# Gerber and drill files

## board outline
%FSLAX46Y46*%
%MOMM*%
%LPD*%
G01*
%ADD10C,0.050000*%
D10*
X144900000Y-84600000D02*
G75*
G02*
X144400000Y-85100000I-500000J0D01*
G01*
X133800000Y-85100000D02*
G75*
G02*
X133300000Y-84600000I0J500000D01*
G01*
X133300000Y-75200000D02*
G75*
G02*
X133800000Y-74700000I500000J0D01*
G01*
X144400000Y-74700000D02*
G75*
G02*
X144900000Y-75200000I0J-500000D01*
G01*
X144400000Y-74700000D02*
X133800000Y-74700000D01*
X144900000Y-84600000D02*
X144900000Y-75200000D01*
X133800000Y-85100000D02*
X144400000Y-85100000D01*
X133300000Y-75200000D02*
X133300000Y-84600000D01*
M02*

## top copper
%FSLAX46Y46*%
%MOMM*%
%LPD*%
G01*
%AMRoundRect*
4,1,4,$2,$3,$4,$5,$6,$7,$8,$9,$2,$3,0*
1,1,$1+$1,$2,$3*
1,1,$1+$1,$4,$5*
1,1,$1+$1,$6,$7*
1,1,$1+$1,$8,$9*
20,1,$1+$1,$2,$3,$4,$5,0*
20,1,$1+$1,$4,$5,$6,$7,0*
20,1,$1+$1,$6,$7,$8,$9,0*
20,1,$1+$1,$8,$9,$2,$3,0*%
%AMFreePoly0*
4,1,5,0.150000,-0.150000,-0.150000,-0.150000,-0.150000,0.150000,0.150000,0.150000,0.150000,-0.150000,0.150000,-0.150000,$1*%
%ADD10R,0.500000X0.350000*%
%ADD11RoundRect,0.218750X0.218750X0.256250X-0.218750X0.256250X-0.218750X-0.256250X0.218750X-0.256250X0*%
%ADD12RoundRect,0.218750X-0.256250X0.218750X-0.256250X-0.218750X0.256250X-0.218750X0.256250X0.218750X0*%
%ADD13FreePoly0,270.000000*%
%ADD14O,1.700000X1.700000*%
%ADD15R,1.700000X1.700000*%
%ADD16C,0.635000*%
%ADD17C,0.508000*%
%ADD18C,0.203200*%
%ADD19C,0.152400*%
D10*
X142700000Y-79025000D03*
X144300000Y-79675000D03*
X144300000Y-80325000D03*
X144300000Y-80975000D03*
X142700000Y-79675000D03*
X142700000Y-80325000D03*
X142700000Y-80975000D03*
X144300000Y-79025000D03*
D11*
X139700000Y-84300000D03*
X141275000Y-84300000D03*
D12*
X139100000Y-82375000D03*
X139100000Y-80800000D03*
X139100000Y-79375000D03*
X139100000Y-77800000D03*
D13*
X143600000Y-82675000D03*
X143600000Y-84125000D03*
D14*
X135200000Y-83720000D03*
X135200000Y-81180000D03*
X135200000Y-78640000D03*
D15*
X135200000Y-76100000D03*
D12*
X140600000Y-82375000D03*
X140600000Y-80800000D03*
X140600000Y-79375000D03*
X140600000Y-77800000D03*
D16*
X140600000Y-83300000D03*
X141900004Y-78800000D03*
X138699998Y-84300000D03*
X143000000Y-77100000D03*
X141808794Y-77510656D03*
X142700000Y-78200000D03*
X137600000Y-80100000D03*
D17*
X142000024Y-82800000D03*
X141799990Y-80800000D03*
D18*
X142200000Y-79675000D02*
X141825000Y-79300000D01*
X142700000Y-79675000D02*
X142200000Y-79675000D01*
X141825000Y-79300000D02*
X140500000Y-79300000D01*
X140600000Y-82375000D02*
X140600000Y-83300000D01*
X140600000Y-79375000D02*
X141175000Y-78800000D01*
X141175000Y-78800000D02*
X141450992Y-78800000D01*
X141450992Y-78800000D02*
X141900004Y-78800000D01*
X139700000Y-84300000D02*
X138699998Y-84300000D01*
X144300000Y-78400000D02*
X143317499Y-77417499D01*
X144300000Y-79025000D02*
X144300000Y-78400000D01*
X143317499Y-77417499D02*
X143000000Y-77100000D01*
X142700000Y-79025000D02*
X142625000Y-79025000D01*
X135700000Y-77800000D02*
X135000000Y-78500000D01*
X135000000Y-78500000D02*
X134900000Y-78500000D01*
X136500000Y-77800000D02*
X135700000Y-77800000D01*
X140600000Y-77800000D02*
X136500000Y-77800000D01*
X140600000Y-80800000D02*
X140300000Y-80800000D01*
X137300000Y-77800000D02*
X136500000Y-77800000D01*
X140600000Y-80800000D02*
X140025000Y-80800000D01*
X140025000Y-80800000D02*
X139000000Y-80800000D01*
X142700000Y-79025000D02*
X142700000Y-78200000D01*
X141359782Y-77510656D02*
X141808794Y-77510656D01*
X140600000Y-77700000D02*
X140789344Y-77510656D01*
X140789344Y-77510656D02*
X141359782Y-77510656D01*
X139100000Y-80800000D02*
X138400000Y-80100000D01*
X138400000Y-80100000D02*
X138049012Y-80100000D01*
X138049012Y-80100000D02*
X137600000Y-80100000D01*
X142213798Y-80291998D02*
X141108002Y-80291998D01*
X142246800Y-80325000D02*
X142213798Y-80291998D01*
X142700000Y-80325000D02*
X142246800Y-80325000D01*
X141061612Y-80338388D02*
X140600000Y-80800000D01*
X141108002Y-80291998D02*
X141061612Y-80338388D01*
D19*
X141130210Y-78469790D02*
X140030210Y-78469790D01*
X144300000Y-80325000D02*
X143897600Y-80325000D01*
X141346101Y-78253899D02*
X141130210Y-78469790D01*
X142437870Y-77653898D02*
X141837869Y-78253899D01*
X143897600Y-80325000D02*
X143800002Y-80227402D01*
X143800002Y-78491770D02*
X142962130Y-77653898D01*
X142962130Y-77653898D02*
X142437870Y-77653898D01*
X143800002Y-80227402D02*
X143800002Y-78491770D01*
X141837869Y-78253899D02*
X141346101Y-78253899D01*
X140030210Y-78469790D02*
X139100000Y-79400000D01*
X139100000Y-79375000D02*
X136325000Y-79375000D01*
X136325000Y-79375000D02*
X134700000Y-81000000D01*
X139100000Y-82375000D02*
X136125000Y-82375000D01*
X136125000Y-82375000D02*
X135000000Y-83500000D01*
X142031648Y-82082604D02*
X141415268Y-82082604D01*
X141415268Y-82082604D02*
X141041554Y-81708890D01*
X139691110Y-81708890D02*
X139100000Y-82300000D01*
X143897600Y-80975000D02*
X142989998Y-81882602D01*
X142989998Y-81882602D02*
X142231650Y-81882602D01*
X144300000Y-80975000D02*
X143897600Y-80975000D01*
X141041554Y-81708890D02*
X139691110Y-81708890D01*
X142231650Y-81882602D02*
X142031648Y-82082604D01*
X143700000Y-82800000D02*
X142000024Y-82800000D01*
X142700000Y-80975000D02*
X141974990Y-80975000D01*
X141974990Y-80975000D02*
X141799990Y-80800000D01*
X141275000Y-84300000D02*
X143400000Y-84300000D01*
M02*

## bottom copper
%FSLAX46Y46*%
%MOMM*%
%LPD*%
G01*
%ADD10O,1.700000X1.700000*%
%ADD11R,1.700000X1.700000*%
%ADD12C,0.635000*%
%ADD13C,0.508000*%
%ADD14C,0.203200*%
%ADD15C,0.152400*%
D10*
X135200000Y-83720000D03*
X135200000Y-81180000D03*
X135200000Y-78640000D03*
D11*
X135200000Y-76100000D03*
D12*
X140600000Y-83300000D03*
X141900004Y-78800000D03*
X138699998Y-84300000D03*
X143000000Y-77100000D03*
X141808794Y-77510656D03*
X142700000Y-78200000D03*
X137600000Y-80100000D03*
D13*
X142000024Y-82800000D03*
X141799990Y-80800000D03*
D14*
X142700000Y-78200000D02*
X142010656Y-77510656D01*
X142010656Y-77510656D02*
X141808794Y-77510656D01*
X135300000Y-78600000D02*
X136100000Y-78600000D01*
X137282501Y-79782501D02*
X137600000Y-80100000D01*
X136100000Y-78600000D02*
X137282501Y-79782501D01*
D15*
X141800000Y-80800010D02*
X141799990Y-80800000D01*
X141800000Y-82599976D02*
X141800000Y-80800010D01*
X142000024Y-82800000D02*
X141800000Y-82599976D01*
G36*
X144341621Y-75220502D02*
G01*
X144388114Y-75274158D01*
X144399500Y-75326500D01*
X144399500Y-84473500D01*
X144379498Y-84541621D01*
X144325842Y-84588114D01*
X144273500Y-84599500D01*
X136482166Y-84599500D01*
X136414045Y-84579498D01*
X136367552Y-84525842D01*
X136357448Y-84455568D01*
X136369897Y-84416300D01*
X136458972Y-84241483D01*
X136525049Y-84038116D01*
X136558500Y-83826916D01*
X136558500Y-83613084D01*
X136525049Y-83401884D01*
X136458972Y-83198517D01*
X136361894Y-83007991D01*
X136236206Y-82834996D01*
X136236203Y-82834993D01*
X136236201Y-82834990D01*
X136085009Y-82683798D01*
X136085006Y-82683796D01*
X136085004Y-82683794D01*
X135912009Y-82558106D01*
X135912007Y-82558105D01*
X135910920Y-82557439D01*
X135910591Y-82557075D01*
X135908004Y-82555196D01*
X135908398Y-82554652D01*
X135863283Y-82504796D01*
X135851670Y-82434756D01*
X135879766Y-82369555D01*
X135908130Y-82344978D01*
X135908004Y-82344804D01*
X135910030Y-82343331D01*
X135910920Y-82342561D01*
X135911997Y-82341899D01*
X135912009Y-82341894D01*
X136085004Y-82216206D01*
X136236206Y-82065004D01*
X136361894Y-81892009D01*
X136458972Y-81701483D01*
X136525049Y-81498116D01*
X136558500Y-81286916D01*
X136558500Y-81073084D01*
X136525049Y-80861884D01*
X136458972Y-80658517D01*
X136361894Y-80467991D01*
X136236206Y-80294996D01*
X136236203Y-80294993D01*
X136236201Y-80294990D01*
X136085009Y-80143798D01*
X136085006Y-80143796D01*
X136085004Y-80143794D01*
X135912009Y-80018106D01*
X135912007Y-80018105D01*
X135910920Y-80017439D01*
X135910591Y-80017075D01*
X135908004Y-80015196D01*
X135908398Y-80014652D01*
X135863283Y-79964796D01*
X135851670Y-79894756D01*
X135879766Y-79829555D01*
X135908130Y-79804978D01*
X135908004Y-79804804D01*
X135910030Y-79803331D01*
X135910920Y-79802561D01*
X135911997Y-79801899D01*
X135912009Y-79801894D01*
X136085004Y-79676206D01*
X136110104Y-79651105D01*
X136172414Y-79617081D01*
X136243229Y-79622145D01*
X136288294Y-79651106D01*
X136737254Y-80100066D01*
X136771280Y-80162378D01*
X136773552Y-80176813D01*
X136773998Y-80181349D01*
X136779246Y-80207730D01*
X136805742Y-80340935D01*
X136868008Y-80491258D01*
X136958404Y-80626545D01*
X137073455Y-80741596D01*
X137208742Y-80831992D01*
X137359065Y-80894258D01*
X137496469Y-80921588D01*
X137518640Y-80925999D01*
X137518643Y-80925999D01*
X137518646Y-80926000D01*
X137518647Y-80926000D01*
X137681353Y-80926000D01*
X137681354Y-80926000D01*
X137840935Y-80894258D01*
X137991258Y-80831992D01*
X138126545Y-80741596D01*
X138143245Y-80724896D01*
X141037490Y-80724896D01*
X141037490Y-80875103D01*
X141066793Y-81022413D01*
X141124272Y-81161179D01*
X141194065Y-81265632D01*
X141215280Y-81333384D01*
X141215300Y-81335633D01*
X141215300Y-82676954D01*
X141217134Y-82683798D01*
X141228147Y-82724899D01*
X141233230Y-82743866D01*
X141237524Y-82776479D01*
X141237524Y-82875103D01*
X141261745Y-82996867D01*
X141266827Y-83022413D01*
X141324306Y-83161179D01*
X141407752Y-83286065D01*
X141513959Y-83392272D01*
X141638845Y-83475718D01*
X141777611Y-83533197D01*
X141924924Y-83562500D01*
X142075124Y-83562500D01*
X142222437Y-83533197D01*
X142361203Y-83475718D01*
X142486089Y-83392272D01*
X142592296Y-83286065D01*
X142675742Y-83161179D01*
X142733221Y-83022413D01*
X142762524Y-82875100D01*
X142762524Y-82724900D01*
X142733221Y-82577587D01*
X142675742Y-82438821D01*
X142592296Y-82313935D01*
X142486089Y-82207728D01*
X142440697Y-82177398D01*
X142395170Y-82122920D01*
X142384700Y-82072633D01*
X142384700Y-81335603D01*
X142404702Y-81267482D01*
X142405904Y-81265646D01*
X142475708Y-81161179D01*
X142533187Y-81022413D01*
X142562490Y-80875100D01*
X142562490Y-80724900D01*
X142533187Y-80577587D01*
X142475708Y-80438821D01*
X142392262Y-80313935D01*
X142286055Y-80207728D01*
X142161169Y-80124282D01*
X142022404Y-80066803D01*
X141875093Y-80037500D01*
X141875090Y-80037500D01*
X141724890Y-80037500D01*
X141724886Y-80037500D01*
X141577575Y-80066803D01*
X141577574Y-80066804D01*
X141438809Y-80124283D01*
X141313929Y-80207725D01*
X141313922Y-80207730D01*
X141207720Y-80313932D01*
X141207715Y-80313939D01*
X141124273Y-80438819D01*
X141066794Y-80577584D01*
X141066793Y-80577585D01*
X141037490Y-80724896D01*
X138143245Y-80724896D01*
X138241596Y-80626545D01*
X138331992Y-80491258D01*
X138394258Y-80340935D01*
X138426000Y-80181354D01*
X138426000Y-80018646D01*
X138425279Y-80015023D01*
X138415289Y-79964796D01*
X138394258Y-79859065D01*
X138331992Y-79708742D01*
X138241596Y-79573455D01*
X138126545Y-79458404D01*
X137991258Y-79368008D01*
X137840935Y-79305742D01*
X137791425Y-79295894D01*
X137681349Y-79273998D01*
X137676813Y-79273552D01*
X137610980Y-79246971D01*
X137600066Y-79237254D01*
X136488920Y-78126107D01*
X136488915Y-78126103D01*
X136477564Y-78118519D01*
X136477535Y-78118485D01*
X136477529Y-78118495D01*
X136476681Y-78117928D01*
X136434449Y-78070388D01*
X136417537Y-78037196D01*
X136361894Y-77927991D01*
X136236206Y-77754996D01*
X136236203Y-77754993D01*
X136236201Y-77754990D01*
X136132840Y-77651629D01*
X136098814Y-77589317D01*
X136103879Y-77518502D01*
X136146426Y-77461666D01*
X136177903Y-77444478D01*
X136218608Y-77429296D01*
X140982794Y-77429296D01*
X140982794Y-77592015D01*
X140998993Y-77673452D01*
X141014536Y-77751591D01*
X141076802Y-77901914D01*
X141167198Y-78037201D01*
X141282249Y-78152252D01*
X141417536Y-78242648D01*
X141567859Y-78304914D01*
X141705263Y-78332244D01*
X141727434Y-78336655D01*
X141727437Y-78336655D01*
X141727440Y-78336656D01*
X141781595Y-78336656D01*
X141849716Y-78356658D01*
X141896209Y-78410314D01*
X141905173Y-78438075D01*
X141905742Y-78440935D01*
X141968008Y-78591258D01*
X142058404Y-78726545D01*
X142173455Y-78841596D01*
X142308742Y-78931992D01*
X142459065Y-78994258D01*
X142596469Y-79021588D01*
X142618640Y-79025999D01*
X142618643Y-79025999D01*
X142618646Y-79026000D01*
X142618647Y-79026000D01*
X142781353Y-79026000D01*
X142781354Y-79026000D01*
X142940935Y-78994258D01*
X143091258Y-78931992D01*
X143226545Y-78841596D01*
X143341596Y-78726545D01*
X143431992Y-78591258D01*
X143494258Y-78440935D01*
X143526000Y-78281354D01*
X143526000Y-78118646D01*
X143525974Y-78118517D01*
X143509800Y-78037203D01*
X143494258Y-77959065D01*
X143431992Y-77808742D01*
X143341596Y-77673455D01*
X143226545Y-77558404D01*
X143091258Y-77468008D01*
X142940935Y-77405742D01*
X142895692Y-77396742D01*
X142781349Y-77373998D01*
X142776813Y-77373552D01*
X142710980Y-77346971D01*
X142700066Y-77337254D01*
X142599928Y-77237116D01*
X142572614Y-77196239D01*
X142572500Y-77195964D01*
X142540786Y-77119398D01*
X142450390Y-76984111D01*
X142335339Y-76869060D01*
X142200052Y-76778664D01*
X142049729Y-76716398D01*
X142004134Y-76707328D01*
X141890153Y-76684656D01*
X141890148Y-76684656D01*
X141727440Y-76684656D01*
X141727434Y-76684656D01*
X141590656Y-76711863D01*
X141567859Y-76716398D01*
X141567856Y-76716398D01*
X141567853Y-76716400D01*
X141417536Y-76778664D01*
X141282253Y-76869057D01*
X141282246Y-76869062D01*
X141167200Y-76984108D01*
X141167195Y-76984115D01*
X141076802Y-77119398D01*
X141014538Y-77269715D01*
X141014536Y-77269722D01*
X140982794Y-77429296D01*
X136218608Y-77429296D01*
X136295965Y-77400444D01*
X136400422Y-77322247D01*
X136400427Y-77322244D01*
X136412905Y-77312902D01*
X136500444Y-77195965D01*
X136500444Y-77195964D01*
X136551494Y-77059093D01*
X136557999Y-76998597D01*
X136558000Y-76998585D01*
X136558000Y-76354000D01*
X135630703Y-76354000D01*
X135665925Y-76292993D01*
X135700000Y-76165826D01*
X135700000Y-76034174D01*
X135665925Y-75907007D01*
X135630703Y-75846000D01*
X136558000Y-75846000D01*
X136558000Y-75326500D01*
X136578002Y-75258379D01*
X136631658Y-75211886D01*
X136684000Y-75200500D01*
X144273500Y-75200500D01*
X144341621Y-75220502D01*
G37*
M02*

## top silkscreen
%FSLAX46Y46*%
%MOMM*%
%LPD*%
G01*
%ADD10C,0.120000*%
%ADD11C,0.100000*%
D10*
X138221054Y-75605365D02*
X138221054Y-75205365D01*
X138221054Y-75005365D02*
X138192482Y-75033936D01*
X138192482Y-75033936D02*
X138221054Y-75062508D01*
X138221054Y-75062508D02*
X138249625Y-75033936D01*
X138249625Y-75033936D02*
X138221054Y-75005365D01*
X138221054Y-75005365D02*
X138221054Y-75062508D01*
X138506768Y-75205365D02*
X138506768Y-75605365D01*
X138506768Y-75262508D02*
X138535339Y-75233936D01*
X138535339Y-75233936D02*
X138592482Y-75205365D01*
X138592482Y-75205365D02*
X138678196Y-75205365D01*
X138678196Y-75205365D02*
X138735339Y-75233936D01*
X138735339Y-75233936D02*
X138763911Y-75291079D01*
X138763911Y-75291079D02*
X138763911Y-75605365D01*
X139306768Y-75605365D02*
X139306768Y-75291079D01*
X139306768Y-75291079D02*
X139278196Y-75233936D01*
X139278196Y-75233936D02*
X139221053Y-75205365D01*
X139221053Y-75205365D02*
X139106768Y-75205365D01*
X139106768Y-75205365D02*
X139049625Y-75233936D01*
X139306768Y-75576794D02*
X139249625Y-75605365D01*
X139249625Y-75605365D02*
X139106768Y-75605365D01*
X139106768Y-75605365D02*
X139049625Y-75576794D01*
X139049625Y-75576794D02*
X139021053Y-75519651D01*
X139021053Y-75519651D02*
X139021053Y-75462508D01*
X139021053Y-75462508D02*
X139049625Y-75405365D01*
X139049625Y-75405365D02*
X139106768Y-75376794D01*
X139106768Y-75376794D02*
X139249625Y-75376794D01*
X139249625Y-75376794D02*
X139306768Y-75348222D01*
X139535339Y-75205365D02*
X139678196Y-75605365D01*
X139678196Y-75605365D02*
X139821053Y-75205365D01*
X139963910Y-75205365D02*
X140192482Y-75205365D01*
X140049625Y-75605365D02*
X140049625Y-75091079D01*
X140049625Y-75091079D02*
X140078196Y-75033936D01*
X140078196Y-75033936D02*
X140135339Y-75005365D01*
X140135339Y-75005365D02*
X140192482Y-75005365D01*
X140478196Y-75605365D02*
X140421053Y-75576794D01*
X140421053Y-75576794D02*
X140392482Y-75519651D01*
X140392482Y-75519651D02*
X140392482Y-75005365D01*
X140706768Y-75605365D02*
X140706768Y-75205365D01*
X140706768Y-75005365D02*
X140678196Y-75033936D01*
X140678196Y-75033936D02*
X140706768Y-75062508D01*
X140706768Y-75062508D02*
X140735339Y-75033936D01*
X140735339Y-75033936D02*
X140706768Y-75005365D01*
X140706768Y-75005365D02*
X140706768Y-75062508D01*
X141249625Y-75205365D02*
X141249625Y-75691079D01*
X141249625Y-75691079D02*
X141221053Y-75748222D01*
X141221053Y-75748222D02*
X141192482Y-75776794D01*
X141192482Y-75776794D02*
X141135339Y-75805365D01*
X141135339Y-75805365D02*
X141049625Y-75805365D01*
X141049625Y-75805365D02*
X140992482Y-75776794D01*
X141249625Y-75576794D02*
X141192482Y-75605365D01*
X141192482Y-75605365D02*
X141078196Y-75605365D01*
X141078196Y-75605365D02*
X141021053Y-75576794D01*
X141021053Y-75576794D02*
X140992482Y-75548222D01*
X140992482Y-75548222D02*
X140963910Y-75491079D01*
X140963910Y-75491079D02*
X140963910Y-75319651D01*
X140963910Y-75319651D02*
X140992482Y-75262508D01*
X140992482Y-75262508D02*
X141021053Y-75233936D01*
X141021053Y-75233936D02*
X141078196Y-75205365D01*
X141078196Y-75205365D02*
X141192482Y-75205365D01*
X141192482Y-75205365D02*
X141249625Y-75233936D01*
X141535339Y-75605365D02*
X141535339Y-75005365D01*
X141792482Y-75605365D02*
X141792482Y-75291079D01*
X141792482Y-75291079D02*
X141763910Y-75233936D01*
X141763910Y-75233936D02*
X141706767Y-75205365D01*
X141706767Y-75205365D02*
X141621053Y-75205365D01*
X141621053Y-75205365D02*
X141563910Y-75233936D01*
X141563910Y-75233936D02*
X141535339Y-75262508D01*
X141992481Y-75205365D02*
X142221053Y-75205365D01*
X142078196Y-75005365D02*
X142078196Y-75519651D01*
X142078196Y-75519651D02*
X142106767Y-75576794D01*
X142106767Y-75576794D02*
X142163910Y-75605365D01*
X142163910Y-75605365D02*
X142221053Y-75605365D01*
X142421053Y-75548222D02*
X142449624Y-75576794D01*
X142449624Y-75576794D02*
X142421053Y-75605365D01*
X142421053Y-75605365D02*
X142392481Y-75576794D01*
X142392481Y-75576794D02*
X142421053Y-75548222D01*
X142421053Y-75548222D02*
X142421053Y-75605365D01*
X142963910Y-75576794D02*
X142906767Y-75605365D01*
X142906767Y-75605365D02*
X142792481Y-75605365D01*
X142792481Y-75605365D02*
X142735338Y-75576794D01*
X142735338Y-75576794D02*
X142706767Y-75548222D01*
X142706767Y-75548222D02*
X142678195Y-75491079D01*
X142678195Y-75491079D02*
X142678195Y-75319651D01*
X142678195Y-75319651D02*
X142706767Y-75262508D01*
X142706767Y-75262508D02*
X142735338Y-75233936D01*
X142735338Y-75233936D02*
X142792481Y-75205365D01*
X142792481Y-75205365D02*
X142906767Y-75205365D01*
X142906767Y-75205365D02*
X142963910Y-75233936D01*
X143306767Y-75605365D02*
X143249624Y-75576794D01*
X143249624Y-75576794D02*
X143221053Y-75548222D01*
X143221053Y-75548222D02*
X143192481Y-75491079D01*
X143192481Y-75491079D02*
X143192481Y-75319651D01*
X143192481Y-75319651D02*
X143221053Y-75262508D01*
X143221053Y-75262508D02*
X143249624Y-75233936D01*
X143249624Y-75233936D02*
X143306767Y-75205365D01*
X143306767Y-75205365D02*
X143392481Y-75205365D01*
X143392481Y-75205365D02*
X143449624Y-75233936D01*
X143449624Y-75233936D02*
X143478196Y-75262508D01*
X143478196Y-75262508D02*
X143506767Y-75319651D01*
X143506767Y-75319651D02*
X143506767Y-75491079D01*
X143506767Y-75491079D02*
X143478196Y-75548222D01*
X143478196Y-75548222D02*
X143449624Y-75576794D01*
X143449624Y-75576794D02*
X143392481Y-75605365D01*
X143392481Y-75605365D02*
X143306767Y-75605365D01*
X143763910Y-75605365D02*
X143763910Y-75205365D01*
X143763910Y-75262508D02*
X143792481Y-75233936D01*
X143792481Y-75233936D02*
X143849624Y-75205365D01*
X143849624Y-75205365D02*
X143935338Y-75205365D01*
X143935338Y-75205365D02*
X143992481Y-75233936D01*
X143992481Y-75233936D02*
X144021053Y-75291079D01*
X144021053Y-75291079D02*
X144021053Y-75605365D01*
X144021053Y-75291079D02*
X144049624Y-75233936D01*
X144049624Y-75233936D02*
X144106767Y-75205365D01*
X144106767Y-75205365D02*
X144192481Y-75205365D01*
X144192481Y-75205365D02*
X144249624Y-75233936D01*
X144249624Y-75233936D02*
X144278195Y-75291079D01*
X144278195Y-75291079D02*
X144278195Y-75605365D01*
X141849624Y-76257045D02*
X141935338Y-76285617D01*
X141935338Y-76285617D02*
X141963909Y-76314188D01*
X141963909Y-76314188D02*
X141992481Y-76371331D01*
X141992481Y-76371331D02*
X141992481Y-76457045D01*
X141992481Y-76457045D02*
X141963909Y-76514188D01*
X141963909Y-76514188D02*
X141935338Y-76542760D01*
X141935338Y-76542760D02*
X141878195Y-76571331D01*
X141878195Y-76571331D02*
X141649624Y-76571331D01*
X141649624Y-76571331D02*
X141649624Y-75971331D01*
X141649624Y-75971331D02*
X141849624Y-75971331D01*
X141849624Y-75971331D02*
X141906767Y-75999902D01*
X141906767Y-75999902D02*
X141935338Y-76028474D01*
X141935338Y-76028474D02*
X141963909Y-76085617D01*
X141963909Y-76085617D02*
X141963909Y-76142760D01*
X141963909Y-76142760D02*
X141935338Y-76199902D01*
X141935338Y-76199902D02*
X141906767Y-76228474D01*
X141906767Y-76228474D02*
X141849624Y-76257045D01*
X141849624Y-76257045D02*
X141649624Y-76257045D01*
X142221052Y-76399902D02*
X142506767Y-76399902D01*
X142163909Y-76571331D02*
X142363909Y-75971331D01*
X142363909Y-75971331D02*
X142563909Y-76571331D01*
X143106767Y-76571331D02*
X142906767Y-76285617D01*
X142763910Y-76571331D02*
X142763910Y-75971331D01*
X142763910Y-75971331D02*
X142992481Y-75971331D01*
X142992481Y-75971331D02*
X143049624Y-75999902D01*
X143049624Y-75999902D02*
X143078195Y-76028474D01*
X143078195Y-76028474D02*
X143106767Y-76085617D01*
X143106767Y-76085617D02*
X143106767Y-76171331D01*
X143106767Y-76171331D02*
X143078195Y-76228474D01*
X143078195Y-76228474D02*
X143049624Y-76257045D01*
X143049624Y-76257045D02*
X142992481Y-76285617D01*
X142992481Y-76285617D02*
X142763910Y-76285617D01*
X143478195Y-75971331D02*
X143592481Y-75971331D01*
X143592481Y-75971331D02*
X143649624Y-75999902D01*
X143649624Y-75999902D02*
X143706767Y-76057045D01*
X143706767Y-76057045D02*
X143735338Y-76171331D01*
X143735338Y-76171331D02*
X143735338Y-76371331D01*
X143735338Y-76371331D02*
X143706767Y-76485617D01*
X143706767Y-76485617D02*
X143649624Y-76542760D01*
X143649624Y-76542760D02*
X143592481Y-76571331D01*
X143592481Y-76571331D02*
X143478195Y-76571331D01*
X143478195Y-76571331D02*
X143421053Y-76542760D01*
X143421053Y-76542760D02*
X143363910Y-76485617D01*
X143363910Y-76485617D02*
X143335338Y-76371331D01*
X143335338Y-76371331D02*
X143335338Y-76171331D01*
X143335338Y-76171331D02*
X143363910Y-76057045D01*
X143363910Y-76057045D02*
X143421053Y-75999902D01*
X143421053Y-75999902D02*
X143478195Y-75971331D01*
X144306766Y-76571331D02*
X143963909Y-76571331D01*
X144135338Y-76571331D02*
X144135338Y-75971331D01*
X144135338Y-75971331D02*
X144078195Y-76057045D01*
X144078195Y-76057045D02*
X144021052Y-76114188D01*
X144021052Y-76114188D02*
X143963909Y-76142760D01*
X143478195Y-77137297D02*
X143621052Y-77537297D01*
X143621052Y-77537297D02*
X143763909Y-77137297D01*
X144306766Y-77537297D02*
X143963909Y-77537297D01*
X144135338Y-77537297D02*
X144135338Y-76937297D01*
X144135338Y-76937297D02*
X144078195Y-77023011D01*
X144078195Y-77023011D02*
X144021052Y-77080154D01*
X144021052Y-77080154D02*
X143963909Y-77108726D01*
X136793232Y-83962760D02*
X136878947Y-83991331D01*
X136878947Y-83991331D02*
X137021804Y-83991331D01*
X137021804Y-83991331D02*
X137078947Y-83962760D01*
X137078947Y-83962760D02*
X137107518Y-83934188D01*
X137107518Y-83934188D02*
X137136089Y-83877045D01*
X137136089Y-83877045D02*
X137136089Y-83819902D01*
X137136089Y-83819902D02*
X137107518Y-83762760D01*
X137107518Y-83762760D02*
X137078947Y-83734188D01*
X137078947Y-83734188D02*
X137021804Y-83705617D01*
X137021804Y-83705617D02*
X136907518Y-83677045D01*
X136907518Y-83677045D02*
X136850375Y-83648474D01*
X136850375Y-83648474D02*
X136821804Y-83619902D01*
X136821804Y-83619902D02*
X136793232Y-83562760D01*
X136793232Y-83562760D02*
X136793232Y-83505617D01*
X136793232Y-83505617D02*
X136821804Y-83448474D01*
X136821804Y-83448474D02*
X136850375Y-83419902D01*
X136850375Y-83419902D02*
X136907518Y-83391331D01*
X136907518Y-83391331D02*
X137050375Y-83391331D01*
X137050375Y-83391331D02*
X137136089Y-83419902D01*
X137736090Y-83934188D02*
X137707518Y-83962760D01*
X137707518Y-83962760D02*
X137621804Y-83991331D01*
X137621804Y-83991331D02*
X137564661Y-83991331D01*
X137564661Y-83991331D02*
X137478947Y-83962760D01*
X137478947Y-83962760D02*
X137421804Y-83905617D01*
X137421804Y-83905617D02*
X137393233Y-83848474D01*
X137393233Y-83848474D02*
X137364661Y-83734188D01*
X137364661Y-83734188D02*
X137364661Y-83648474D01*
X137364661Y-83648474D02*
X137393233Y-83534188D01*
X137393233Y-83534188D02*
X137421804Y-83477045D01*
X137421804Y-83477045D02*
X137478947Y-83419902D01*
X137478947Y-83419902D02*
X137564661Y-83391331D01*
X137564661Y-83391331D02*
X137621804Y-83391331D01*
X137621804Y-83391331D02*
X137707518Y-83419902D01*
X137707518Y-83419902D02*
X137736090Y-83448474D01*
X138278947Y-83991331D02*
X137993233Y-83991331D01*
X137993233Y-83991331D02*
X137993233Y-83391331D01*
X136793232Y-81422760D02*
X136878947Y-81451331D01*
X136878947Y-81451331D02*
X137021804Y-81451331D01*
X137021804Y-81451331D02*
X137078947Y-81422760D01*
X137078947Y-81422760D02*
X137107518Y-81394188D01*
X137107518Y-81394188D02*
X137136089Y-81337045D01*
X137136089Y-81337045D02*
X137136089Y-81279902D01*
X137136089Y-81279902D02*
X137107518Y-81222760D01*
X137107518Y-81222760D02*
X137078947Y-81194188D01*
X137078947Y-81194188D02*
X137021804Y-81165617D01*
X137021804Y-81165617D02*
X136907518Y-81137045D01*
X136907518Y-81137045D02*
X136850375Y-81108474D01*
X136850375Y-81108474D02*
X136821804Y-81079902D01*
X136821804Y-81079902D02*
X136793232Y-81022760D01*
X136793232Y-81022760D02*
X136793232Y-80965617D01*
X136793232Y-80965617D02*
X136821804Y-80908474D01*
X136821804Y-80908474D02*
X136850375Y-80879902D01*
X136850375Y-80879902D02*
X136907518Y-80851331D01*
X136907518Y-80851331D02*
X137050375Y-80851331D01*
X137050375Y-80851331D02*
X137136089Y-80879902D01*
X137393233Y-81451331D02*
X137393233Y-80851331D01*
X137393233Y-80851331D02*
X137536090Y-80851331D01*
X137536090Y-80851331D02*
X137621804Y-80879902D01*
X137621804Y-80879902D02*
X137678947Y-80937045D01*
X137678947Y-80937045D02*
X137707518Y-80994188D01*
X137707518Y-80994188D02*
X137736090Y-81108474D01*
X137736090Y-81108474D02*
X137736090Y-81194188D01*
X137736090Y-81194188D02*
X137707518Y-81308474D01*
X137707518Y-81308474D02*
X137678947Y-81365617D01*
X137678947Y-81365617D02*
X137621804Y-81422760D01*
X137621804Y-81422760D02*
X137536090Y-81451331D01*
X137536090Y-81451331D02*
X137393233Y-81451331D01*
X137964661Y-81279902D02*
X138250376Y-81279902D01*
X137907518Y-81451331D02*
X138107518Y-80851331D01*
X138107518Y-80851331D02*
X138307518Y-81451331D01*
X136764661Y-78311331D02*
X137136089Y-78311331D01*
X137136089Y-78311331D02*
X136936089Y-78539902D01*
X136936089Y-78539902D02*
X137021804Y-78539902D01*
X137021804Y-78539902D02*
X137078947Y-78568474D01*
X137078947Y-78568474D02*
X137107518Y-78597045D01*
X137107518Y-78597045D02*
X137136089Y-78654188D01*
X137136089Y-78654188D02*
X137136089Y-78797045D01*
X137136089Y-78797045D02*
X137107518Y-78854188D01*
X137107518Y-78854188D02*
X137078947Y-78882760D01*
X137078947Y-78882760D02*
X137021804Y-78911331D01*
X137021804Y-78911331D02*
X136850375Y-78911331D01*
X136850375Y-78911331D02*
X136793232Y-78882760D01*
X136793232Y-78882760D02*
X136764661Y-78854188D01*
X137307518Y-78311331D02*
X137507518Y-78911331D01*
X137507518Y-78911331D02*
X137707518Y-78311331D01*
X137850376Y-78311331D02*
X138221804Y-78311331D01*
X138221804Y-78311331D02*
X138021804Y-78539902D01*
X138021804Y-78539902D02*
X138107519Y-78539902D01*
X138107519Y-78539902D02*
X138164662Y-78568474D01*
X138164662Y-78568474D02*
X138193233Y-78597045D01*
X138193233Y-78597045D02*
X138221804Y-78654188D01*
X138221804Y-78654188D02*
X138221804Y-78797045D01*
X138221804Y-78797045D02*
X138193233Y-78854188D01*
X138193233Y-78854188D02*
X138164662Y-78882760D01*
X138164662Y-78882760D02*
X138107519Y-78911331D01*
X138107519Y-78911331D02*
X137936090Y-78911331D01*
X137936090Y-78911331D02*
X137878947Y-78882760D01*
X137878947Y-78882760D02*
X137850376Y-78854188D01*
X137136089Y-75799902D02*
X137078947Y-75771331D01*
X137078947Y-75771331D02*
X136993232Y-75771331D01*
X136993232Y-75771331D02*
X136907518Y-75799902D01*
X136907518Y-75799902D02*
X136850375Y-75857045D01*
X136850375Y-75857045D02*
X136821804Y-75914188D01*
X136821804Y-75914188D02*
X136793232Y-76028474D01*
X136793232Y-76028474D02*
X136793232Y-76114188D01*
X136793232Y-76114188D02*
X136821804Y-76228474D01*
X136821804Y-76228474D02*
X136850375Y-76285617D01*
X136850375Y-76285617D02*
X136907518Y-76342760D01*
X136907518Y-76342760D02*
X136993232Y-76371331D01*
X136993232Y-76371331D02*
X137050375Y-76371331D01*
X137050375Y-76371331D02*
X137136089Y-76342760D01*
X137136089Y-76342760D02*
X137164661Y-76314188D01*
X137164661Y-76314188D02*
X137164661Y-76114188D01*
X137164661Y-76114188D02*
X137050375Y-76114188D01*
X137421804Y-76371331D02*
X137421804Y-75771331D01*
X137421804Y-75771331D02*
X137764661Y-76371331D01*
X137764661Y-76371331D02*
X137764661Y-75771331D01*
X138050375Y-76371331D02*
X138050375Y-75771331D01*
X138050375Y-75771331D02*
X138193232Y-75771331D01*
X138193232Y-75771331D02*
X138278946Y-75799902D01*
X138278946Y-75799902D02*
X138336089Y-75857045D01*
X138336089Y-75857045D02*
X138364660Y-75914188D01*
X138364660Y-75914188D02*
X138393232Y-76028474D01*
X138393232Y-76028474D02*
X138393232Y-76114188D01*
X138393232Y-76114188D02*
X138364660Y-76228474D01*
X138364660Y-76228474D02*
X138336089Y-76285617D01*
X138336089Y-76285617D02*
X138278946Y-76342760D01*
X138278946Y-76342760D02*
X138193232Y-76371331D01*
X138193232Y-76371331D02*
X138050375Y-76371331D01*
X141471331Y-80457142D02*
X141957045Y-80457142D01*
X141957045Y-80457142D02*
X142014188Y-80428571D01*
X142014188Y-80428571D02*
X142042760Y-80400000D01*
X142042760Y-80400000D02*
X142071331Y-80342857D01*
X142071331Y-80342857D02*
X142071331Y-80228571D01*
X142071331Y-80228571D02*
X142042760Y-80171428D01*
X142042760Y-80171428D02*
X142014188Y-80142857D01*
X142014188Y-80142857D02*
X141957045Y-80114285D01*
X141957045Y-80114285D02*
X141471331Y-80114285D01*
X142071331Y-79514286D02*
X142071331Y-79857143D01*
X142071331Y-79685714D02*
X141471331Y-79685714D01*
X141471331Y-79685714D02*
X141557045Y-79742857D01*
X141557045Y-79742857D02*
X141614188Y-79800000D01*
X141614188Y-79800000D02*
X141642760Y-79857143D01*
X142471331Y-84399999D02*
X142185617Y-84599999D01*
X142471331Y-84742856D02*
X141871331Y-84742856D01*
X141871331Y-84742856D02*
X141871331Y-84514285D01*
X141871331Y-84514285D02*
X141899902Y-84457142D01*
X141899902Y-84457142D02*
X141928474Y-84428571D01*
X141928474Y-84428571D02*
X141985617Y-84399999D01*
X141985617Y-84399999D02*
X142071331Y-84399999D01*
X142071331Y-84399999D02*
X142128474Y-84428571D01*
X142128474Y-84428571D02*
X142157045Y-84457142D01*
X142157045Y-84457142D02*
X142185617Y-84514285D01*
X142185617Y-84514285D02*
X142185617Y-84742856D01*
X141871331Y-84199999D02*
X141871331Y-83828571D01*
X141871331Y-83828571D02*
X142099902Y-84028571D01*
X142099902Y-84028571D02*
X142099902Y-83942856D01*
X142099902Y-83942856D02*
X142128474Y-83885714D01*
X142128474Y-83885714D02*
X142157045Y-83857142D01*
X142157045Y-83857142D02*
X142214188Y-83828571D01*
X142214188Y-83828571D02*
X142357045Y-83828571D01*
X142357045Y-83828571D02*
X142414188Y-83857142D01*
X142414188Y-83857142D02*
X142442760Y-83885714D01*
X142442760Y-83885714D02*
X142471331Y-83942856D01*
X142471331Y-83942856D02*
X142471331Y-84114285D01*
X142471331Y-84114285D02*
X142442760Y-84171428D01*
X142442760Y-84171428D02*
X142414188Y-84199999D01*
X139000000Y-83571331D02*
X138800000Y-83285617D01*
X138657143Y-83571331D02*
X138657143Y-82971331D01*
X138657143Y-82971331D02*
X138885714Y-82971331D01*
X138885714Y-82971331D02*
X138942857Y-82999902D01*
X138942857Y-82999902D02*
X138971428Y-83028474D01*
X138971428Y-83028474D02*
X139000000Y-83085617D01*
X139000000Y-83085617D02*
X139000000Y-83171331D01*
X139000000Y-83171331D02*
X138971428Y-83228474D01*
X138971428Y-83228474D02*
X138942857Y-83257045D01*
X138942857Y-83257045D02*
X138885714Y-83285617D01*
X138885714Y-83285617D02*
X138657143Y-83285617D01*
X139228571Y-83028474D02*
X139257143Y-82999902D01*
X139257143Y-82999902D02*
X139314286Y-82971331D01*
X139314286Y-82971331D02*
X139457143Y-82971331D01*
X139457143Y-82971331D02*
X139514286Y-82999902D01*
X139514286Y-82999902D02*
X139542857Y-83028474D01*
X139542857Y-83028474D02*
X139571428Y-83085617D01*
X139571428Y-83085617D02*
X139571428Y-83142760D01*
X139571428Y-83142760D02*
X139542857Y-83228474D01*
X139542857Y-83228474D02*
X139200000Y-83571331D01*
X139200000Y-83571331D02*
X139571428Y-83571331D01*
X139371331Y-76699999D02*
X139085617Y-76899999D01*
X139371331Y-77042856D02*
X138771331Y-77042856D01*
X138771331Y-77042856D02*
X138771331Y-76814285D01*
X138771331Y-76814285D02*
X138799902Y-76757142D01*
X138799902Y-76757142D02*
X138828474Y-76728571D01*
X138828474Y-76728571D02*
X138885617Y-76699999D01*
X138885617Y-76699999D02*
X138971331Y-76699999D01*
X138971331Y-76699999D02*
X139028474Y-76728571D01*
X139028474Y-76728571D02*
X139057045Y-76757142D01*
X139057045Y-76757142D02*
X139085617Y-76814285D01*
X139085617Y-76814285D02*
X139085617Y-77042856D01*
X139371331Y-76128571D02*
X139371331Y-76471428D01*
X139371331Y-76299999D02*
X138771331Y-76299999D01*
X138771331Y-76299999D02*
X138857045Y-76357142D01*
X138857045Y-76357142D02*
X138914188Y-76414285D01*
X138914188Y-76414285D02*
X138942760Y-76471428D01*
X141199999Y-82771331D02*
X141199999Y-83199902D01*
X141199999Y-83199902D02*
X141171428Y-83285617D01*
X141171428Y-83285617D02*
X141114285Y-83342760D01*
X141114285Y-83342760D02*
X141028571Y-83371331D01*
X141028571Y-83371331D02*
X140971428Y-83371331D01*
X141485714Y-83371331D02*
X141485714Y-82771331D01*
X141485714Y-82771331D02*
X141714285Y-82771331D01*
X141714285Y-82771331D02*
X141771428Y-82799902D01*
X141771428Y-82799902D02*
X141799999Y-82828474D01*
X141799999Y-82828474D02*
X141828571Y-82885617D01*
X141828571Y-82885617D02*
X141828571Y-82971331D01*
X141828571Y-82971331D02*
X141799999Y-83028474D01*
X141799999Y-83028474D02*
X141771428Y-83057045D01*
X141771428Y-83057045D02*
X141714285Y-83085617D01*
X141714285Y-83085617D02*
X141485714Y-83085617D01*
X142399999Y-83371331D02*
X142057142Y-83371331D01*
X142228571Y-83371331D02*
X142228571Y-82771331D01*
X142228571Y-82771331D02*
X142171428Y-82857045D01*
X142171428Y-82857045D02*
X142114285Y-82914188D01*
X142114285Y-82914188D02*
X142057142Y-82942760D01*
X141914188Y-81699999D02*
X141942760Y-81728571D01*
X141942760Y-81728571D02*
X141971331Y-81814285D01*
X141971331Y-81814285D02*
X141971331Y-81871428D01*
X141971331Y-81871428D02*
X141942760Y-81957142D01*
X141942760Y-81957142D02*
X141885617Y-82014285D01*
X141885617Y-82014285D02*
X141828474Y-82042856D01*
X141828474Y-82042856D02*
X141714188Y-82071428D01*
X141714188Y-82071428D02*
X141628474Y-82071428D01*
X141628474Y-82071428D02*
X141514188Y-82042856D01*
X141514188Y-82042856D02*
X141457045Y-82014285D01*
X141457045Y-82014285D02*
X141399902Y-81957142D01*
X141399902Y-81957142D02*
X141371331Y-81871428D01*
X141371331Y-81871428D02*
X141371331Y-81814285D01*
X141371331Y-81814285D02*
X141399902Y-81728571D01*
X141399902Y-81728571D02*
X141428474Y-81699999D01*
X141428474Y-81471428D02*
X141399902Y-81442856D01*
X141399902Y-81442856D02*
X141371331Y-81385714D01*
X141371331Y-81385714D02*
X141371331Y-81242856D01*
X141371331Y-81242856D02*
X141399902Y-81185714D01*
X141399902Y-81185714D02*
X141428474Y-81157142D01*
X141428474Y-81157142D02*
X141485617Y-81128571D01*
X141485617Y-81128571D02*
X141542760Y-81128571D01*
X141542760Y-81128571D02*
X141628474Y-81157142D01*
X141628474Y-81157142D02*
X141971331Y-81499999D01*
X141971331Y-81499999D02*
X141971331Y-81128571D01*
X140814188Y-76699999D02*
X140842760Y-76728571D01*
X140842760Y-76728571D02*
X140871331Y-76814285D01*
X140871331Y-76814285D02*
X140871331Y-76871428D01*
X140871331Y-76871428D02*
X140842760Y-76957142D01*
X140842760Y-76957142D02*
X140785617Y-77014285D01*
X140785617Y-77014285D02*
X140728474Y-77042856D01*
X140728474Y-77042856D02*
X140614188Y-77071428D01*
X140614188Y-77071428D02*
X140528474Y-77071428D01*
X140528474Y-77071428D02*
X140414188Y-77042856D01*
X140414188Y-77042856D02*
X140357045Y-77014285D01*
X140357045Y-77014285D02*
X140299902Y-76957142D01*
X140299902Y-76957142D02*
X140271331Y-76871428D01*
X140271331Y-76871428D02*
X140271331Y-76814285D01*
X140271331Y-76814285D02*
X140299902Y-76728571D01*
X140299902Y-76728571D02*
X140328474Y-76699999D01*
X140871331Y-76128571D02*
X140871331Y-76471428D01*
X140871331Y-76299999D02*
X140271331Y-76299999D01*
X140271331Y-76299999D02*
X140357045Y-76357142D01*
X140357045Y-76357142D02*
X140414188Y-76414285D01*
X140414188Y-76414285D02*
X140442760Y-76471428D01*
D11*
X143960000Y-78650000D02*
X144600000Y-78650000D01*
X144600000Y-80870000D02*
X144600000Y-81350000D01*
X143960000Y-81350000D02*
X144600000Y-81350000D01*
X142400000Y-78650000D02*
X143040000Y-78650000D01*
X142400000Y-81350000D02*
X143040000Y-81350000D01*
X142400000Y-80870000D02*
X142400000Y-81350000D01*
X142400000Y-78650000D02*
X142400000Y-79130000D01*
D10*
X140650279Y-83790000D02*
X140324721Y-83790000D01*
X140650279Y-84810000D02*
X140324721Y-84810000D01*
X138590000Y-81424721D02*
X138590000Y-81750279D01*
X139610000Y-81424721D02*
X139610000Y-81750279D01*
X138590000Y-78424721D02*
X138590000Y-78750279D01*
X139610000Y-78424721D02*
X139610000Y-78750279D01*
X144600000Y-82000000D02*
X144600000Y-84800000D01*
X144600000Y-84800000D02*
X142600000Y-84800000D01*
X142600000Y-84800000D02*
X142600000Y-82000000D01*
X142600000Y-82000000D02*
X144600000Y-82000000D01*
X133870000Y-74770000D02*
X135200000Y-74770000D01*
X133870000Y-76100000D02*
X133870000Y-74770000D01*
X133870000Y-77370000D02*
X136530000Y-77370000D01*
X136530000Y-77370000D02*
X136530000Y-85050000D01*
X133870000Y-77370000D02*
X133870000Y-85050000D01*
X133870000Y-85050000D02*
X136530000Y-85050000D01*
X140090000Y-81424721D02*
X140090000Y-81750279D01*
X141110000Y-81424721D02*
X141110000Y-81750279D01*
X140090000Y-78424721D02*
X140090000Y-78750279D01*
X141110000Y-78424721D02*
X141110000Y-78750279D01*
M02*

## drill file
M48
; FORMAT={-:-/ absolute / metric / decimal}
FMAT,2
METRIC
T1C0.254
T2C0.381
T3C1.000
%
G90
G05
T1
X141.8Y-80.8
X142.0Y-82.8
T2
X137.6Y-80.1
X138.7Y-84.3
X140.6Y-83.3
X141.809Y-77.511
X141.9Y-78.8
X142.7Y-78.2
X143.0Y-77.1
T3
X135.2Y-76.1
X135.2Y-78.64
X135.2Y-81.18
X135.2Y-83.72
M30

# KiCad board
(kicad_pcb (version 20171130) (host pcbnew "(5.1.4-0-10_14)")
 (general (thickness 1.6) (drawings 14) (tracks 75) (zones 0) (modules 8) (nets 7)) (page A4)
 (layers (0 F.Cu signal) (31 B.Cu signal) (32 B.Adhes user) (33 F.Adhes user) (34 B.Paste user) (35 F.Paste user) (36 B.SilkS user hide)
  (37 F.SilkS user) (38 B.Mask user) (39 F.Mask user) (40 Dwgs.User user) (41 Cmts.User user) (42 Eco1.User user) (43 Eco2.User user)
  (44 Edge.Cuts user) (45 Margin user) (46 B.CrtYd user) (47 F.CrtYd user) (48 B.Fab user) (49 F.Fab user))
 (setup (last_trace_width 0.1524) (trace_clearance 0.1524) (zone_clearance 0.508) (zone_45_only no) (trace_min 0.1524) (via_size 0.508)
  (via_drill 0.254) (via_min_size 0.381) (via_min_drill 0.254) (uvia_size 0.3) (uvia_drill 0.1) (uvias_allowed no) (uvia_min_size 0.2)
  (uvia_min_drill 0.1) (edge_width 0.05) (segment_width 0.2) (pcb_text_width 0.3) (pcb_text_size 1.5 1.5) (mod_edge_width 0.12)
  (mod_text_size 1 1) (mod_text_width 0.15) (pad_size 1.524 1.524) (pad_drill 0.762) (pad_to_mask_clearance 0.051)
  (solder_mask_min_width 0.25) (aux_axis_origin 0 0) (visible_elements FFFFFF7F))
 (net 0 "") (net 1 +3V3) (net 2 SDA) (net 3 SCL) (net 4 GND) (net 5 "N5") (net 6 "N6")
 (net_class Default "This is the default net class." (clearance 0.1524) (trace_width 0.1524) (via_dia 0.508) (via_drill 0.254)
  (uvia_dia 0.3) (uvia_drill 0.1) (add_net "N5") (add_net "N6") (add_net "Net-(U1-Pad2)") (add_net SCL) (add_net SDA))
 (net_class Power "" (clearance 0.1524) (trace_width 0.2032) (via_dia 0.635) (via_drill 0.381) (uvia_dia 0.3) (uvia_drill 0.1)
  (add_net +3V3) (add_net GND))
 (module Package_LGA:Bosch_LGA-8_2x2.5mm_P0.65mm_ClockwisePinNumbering (layer F.Cu) (at 143.5 80 270)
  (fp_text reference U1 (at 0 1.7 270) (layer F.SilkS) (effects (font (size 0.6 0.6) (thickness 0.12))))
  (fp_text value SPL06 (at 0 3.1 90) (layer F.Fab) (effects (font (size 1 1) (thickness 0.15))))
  (fp_line (start -1.35 -0.46) (end -1.35 -1.1) (layer F.SilkS) (width 0.1))
  (fp_line (start 0.87 -1.1) (end 1.35 -1.1) (layer F.SilkS) (width 0.1))
  (fp_line (start 1.35 -0.46) (end 1.35 -1.1) (layer F.SilkS) (width 0.1))
  (fp_line (start -1.35 1.1) (end -1.35 0.46) (layer F.SilkS) (width 0.1))
  (fp_line (start 1.35 1.1) (end 1.35 0.46) (layer F.SilkS) (width 0.1))
  (fp_line (start 0.87 1.1) (end 1.35 1.1) (layer F.SilkS) (width 0.1))
  (fp_line (start -1.35 1.1) (end -0.87 1.1) (layer F.SilkS) (width 0.1))
  (pad 8 smd rect (at -0.975 0.8) (size 0.5 0.35) (layers F.Cu F.Paste F.Mask) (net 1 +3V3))
  (pad 2 smd rect (at -0.325 -0.8) (size 0.5 0.35) (layers F.Cu F.Paste F.Mask))
  (pad 3 smd rect (at 0.325 -0.8) (size 0.5 0.35) (layers F.Cu F.Paste F.Mask) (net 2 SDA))
  (pad 4 smd rect (at 0.975 -0.8) (size 0.5 0.35) (layers F.Cu F.Paste F.Mask) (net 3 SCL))
  (pad 7 smd rect (at -0.325 0.8) (size 0.5 0.35) (layers F.Cu F.Paste F.Mask) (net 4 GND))
  (pad 6 smd rect (at 0.325 0.8) (size 0.5 0.35) (layers F.Cu F.Paste F.Mask) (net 1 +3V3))
  (pad 5 smd rect (at 0.975 0.8) (size 0.5 0.35) (layers F.Cu F.Paste F.Mask) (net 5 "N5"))
  (pad 1 smd rect (at -0.975 -0.8) (size 0.5 0.35) (layers F.Cu F.Paste F.Mask) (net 4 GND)))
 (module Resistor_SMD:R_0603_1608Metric (layer F.Cu) (at 140.4875 84.3 180)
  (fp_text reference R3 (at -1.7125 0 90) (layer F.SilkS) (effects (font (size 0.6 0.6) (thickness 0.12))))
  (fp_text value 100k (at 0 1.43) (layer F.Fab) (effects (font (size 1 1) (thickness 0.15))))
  (fp_line (start -0.162779 0.51) (end 0.162779 0.51) (layer F.SilkS) (width 0.12))
  (fp_line (start -0.162779 -0.51) (end 0.162779 -0.51) (layer F.SilkS) (width 0.12))
  (pad 2 smd roundrect (at 0.7875 0 180) (size 0.875 0.95) (layers F.Cu F.Paste F.Mask) (roundrect_rratio 0.25) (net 4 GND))
  (pad 1 smd roundrect (at -0.7875 0 180) (size 0.875 0.95) (layers F.Cu F.Paste F.Mask) (roundrect_rratio 0.25) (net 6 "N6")))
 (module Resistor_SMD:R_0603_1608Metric (layer F.Cu) (at 139.1 81.5875 270)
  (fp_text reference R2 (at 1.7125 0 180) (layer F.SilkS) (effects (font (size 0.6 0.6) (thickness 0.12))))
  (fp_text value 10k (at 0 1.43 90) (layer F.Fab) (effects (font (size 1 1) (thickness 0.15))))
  (fp_line (start -0.162779 0.51) (end 0.162779 0.51) (layer F.SilkS) (width 0.12))
  (fp_line (start -0.162779 -0.51) (end 0.162779 -0.51) (layer F.SilkS) (width 0.12))
  (pad 2 smd roundrect (at 0.7875 0 270) (size 0.875 0.95) (layers F.Cu F.Paste F.Mask) (roundrect_rratio 0.25) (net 3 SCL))
  (pad 1 smd roundrect (at -0.7875 0 270) (size 0.875 0.95) (layers F.Cu F.Paste F.Mask) (roundrect_rratio 0.25) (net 1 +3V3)))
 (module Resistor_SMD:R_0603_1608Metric (layer F.Cu) (at 139.1 78.5875 270)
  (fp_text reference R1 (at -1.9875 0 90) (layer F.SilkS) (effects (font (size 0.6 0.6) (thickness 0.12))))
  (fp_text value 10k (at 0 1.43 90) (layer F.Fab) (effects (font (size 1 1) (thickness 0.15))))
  (fp_line (start -0.162779 0.51) (end 0.162779 0.51) (layer F.SilkS) (width 0.12))
  (fp_line (start -0.162779 -0.51) (end 0.162779 -0.51) (layer F.SilkS) (width 0.12))
  (pad 2 smd roundrect (at 0.7875 0 270) (size 0.875 0.95) (layers F.Cu F.Paste F.Mask) (roundrect_rratio 0.25) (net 2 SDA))
  (pad 1 smd roundrect (at -0.7875 0 270) (size 0.875 0.95) (layers F.Cu F.Paste F.Mask) (roundrect_rratio 0.25) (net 1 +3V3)))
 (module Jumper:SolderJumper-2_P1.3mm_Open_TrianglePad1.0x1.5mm (layer F.Cu) (at 143.6 83.4 270)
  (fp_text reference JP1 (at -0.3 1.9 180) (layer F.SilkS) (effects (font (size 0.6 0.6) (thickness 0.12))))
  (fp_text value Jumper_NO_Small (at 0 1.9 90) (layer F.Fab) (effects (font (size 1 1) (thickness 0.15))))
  (fp_line (start -1.4 -1) (end 1.4 -1) (layer F.SilkS) (width 0.12))
  (fp_line (start 1.4 -1) (end 1.4 1) (layer F.SilkS) (width 0.12))
  (fp_line (start 1.4 1) (end -1.4 1) (layer F.SilkS) (width 0.12))
  (fp_line (start -1.4 1) (end -1.4 -1) (layer F.SilkS) (width 0.12))
  (pad 1 smd custom (at -0.725 0 270) (size 0.3 0.3) (layers F.Cu F.Mask) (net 5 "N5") (zone_connect 2)
   (options (clearance outline) (anchor rect)) (primitives))
  (pad 2 smd custom (at 0.725 0 270) (size 0.3 0.3) (layers F.Cu F.Mask) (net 6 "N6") (zone_connect 2)
   (options (clearance outline) (anchor rect)) (primitives)))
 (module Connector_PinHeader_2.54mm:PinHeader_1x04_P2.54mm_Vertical (layer F.Cu) (at 135.2 76.1)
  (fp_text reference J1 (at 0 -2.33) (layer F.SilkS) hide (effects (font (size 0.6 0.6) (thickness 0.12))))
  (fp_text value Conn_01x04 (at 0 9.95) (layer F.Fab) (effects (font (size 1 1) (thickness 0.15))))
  (fp_line (start -1.33 -1.33) (end 0 -1.33) (layer F.SilkS) (width 0.12))
  (fp_line (start -1.33 0) (end -1.33 -1.33) (layer F.SilkS) (width 0.12))
  (fp_line (start -1.33 1.27) (end 1.33 1.27) (layer F.SilkS) (width 0.12))
  (fp_line (start 1.33 1.27) (end 1.33 8.95) (layer F.SilkS) (width 0.12))
  (fp_line (start -1.33 1.27) (end -1.33 8.95) (layer F.SilkS) (width 0.12))
  (fp_line (start -1.33 8.95) (end 1.33 8.95) (layer F.SilkS) (width 0.12))
  (pad 4 thru_hole oval (at 0 7.62) (size 1.7 1.7) (drill 1) (layers *.Cu *.Mask) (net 3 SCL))
  (pad 3 thru_hole oval (at 0 5.08) (size 1.7 1.7) (drill 1) (layers *.Cu *.Mask) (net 2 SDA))
  (pad 2 thru_hole oval (at 0 2.54) (size 1.7 1.7) (drill 1) (layers *.Cu *.Mask) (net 1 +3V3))
  (pad 1 thru_hole rect (at 0 0) (size 1.7 1.7) (drill 1) (layers *.Cu *.Mask) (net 4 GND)))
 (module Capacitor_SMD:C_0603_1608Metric (layer F.Cu) (at 140.6 81.5875 270)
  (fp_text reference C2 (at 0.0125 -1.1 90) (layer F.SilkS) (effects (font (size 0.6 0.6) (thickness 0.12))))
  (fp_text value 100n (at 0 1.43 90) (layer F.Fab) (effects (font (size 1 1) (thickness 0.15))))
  (fp_line (start -0.162779 0.51) (end 0.162779 0.51) (layer F.SilkS) (width 0.12))
  (fp_line (start -0.162779 -0.51) (end 0.162779 -0.51) (layer F.SilkS) (width 0.12))
  (pad 2 smd roundrect (at 0.7875 0 270) (size 0.875 0.95) (layers F.Cu F.Paste F.Mask) (roundrect_rratio 0.25) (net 4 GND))
  (pad 1 smd roundrect (at -0.7875 0 270) (size 0.875 0.95) (layers F.Cu F.Paste F.Mask) (roundrect_rratio 0.25) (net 1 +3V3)))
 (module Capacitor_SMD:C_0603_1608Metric (layer F.Cu) (at 140.6 78.5875 270)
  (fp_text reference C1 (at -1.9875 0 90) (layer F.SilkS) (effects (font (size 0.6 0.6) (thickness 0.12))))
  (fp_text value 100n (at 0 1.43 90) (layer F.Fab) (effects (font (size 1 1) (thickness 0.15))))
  (fp_line (start -0.162779 0.51) (end 0.162779 0.51) (layer F.SilkS) (width 0.12))
  (fp_line (start -0.162779 -0.51) (end 0.162779 -0.51) (layer F.SilkS) (width 0.12))
  (pad 2 smd roundrect (at 0.7875 0 270) (size 0.875 0.95) (layers F.Cu F.Paste F.Mask) (roundrect_rratio 0.25) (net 4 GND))
  (pad 1 smd roundrect (at -0.7875 0 270) (size 0.875 0.95) (layers F.Cu F.Paste F.Mask) (roundrect_rratio 0.25) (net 1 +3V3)))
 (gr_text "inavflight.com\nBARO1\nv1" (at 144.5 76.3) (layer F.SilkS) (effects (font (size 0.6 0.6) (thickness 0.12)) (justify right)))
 (gr_arc (start 144.4 84.6) (end 144.4 85.1) (angle -90) (layer Edge.Cuts) (width 0.05))
 (gr_arc (start 133.8 84.6) (end 133.3 84.6) (angle -90) (layer Edge.Cuts) (width 0.05))
 (gr_arc (start 133.8 75.2) (end 133.8 74.7) (angle -90) (layer Edge.Cuts) (width 0.05))
 (gr_arc (start 144.4 75.2) (end 144.9 75.2) (angle -90) (layer Edge.Cuts) (width 0.05))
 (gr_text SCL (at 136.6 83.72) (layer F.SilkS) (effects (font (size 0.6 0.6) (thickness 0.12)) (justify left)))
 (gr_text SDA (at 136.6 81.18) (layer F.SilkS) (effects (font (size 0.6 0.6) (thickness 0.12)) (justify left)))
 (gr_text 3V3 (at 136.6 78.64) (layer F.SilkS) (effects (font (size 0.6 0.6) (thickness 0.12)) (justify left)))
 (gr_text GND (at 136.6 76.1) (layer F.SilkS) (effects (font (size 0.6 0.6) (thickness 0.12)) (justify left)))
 (gr_line (start 144.4 74.7) (end 133.8 74.7) (layer Edge.Cuts) (width 0.05))
 (gr_line (start 144.9 84.6) (end 144.9 75.2) (layer Edge.Cuts) (width 0.05))
 (gr_line (start 133.8 85.1) (end 144.4 85.1) (layer Edge.Cuts) (width 0.05))
 (gr_line (start 133.3 75.2) (end 133.3 84.6) (layer Edge.Cuts) (width 0.05))
 (segment (start 142.2 79.675) (end 141.825 79.3) (width 0.2032) (layer F.Cu) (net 4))
 (segment (start 142.7 79.675) (end 142.2 79.675) (width 0.2032) (layer F.Cu) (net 4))
 (segment (start 141.825 79.3) (end 140.5 79.3) (width 0.2032) (layer F.Cu) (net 4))
 (via (at 140.6 83.3) (size 0.635) (drill 0.381) (layers F.Cu B.Cu) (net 4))
 (segment (start 140.6 82.375) (end 140.6 83.3) (width 0.2032) (layer F.Cu) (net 4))
 (via (at 141.900004 78.8) (size 0.635) (drill 0.381) (layers F.Cu B.Cu) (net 4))
 (segment (start 140.6 79.375) (end 141.175 78.8) (width 0.2032) (layer F.Cu) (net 4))
 (segment (start 141.175 78.8) (end 141.450992 78.8) (width 0.2032) (layer F.Cu) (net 4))
 (segment (start 141.450992 78.8) (end 141.900004 78.8) (width 0.2032) (layer F.Cu) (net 4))
 (via (at 138.699998 84.3) (size 0.635) (drill 0.381) (layers F.Cu B.Cu) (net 4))
 (segment (start 139.7 84.3) (end 138.699998 84.3) (width 0.2032) (layer F.Cu) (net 4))
 (segment (start 144.3 78.4) (end 143.317499 77.417499) (width 0.2032) (layer F.Cu) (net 4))
 (segment (start 144.3 79.025) (end 144.3 78.4) (width 0.2032) (layer F.Cu) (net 4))
 (segment (start 143.317499 77.417499) (end 143 77.1) (width 0.2032) (layer F.Cu) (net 4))
 (via (at 143 77.1) (size 0.635) (drill 0.381) (layers F.Cu B.Cu) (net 4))
 (segment (start 142.7 79.025) (end 142.625 79.025) (width 0.2032) (layer F.Cu) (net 1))
 (segment (start 135.7 77.8) (end 135 78.5) (width 0.2032) (layer F.Cu) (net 1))
 (segment (start 135 78.5) (end 134.9 78.5) (width 0.2032) (layer F.Cu) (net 1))
 (segment (start 136.5 77.8) (end 135.7 77.8) (width 0.2032) (layer F.Cu) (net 1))
 (segment (start 140.6 77.8) (end 136.5 77.8) (width 0.2032) (layer F.Cu) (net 1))
 (segment (start 140.6 80.8) (end 140.3 80.8) (width 0.2032) (layer F.Cu) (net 1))
 (segment (start 137.3 77.8) (end 136.5 77.8) (width 0.2032) (layer F.Cu) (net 1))
 (segment (start 140.6 80.8) (end 140.025 80.8) (width 0.2032) (layer F.Cu) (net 1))
 (segment (start 140.025 80.8) (end 139 80.8) (width 0.2032) (layer F.Cu) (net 1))
 (segment (start 142.7 79.025) (end 142.7 78.2) (width 0.2032) (layer F.Cu) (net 1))
 (segment (start 142.7 78.2) (end 142.010656 77.510656) (width 0.2032) (layer B.Cu) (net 1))
 (via (at 141.808794 77.510656) (size 0.635) (drill 0.381) (layers F.Cu B.Cu) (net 1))
 (segment (start 141.359782 77.510656) (end 141.808794 77.510656) (width 0.2032) (layer F.Cu) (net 1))
 (segment (start 140.6 77.7) (end 140.789344 77.510656) (width 0.2032) (layer F.Cu) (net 1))
 (segment (start 140.789344 77.510656) (end 141.359782 77.510656) (width 0.2032) (layer F.Cu) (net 1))
 (via (at 142.7 78.2) (size 0.635) (drill 0.381) (layers F.Cu B.Cu) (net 1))
 (segment (start 142.010656 77.510656) (end 141.808794 77.510656) (width 0.2032) (layer B.Cu) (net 1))
 (segment (start 135.3 78.6) (end 136.1 78.6) (width 0.2032) (layer B.Cu) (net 1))
 (segment (start 139.1 80.8) (end 138.4 80.1) (width 0.2032) (layer F.Cu) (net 1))
 (segment (start 138.4 80.1) (end 138.049012 80.1) (width 0.2032) (layer F.Cu) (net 1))
 (segment (start 137.282501 79.782501) (end 137.6 80.1) (width 0.2032) (layer B.Cu) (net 1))
 (via (at 137.6 80.1) (size 0.635) (drill 0.381) (layers F.Cu B.Cu) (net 1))
 (segment (start 138.049012 80.1) (end 137.6 80.1) (width 0.2032) (layer F.Cu) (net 1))
 (segment (start 136.1 78.6) (end 137.282501 79.782501) (width 0.2032) (layer B.Cu) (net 1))
 (segment (start 142.213798 80.291998) (end 141.108002 80.291998) (width 0.2032) (layer F.Cu) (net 1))
 (segment (start 142.2468 80.325) (end 142.213798 80.291998) (width 0.2032) (layer F.Cu) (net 1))
 (segment (start 142.7 80.325) (end 142.2468 80.325) (width 0.2032) (layer F.Cu) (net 1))
 (segment (start 141.061612 80.338388) (end 140.6 80.8) (width 0.2032) (layer F.Cu) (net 1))
 (segment (start 141.108002 80.291998) (end 141.061612 80.338388) (width 0.2032) (layer F.Cu) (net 1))
 (segment (start 141.13021 78.46979) (end 140.03021 78.46979) (width 0.1524) (layer F.Cu) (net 2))
 (segment (start 144.3 80.325) (end 143.8976 80.325) (width 0.1524) (layer F.Cu) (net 2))
 (segment (start 141.346101 78.253899) (end 141.13021 78.46979) (width 0.1524) (layer F.Cu) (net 2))
 (segment (start 142.43787 77.653898) (end 141.837869 78.253899) (width 0.1524) (layer F.Cu) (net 2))
 (segment (start 143.8976 80.325) (end 143.800002 80.227402) (width 0.1524) (layer F.Cu) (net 2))
 (segment (start 143.800002 78.49177) (end 142.96213 77.653898) (width 0.1524) (layer F.Cu) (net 2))
 (segment (start 142.96213 77.653898) (end 142.43787 77.653898) (width 0.1524) (layer F.Cu) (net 2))
 (segment (start 143.800002 80.227402) (end 143.800002 78.49177) (width 0.1524) (layer F.Cu) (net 2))
 (segment (start 141.837869 78.253899) (end 141.346101 78.253899) (width 0.1524) (layer F.Cu) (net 2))
 (segment (start 140.03021 78.46979) (end 139.1 79.4) (width 0.1524) (layer F.Cu) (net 2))
 (segment (start 139.1 79.375) (end 136.325 79.375) (width 0.1524) (layer F.Cu) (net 2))
 (segment (start 136.325 79.375) (end 134.7 81) (width 0.1524) (layer F.Cu) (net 2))
 (segment (start 139.1 82.375) (end 136.125 82.375) (width 0.1524) (layer F.Cu) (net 3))
 (segment (start 136.125 82.375) (end 135 83.5) (width 0.1524) (layer F.Cu) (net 3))
 (segment (start 142.031648 82.082604) (end 141.415268 82.082604) (width 0.1524) (layer F.Cu) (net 3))
 (segment (start 141.415268 82.082604) (end 141.041554 81.70889) (width 0.1524) (layer F.Cu) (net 3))
 (segment (start 139.69111 81.70889) (end 139.1 82.3) (width 0.1524) (layer F.Cu) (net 3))
 (segment (start 143.8976 80.975) (end 142.989998 81.882602) (width 0.1524) (layer F.Cu) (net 3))
 (segment (start 142.989998 81.882602) (end 142.23165 81.882602) (width 0.1524) (layer F.Cu) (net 3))
 (segment (start 144.3 80.975) (end 143.8976 80.975) (width 0.1524) (layer F.Cu) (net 3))
 (segment (start 141.041554 81.70889) (end 139.69111 81.70889) (width 0.1524) (layer F.Cu) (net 3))
 (segment (start 142.23165 81.882602) (end 142.031648 82.082604) (width 0.1524) (layer F.Cu) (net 3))
 (via (at 142.000024 82.8) (size 0.508) (drill 0.254) (layers F.Cu B.Cu) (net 5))
 (segment (start 143.7 82.8) (end 142.000024 82.8) (width 0.1524) (layer F.Cu) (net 5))
 (via (at 141.79999 80.8) (size 0.508) (drill 0.254) (layers F.Cu B.Cu) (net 5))
 (segment (start 142.7 80.975) (end 141.97499 80.975) (width 0.1524) (layer F.Cu) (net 5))
 (segment (start 141.97499 80.975) (end 141.79999 80.8) (width 0.1524) (layer F.Cu) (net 5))
 (segment (start 141.8 80.80001) (end 141.79999 80.8) (width 0.1524) (layer B.Cu) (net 5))
 (segment (start 141.8 82.599976) (end 141.8 80.80001) (width 0.1524) (layer B.Cu) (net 5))
 (segment (start 142.000024 82.8) (end 141.8 82.599976) (width 0.1524) (layer B.Cu) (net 5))
 (segment (start 141.275 84.3) (end 143.4 84.3) (width 0.1524) (layer F.Cu) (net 6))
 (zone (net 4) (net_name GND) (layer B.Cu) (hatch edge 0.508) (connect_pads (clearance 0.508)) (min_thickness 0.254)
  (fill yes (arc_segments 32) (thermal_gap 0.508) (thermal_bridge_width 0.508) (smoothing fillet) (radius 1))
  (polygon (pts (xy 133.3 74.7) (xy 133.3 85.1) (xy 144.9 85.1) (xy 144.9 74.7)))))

